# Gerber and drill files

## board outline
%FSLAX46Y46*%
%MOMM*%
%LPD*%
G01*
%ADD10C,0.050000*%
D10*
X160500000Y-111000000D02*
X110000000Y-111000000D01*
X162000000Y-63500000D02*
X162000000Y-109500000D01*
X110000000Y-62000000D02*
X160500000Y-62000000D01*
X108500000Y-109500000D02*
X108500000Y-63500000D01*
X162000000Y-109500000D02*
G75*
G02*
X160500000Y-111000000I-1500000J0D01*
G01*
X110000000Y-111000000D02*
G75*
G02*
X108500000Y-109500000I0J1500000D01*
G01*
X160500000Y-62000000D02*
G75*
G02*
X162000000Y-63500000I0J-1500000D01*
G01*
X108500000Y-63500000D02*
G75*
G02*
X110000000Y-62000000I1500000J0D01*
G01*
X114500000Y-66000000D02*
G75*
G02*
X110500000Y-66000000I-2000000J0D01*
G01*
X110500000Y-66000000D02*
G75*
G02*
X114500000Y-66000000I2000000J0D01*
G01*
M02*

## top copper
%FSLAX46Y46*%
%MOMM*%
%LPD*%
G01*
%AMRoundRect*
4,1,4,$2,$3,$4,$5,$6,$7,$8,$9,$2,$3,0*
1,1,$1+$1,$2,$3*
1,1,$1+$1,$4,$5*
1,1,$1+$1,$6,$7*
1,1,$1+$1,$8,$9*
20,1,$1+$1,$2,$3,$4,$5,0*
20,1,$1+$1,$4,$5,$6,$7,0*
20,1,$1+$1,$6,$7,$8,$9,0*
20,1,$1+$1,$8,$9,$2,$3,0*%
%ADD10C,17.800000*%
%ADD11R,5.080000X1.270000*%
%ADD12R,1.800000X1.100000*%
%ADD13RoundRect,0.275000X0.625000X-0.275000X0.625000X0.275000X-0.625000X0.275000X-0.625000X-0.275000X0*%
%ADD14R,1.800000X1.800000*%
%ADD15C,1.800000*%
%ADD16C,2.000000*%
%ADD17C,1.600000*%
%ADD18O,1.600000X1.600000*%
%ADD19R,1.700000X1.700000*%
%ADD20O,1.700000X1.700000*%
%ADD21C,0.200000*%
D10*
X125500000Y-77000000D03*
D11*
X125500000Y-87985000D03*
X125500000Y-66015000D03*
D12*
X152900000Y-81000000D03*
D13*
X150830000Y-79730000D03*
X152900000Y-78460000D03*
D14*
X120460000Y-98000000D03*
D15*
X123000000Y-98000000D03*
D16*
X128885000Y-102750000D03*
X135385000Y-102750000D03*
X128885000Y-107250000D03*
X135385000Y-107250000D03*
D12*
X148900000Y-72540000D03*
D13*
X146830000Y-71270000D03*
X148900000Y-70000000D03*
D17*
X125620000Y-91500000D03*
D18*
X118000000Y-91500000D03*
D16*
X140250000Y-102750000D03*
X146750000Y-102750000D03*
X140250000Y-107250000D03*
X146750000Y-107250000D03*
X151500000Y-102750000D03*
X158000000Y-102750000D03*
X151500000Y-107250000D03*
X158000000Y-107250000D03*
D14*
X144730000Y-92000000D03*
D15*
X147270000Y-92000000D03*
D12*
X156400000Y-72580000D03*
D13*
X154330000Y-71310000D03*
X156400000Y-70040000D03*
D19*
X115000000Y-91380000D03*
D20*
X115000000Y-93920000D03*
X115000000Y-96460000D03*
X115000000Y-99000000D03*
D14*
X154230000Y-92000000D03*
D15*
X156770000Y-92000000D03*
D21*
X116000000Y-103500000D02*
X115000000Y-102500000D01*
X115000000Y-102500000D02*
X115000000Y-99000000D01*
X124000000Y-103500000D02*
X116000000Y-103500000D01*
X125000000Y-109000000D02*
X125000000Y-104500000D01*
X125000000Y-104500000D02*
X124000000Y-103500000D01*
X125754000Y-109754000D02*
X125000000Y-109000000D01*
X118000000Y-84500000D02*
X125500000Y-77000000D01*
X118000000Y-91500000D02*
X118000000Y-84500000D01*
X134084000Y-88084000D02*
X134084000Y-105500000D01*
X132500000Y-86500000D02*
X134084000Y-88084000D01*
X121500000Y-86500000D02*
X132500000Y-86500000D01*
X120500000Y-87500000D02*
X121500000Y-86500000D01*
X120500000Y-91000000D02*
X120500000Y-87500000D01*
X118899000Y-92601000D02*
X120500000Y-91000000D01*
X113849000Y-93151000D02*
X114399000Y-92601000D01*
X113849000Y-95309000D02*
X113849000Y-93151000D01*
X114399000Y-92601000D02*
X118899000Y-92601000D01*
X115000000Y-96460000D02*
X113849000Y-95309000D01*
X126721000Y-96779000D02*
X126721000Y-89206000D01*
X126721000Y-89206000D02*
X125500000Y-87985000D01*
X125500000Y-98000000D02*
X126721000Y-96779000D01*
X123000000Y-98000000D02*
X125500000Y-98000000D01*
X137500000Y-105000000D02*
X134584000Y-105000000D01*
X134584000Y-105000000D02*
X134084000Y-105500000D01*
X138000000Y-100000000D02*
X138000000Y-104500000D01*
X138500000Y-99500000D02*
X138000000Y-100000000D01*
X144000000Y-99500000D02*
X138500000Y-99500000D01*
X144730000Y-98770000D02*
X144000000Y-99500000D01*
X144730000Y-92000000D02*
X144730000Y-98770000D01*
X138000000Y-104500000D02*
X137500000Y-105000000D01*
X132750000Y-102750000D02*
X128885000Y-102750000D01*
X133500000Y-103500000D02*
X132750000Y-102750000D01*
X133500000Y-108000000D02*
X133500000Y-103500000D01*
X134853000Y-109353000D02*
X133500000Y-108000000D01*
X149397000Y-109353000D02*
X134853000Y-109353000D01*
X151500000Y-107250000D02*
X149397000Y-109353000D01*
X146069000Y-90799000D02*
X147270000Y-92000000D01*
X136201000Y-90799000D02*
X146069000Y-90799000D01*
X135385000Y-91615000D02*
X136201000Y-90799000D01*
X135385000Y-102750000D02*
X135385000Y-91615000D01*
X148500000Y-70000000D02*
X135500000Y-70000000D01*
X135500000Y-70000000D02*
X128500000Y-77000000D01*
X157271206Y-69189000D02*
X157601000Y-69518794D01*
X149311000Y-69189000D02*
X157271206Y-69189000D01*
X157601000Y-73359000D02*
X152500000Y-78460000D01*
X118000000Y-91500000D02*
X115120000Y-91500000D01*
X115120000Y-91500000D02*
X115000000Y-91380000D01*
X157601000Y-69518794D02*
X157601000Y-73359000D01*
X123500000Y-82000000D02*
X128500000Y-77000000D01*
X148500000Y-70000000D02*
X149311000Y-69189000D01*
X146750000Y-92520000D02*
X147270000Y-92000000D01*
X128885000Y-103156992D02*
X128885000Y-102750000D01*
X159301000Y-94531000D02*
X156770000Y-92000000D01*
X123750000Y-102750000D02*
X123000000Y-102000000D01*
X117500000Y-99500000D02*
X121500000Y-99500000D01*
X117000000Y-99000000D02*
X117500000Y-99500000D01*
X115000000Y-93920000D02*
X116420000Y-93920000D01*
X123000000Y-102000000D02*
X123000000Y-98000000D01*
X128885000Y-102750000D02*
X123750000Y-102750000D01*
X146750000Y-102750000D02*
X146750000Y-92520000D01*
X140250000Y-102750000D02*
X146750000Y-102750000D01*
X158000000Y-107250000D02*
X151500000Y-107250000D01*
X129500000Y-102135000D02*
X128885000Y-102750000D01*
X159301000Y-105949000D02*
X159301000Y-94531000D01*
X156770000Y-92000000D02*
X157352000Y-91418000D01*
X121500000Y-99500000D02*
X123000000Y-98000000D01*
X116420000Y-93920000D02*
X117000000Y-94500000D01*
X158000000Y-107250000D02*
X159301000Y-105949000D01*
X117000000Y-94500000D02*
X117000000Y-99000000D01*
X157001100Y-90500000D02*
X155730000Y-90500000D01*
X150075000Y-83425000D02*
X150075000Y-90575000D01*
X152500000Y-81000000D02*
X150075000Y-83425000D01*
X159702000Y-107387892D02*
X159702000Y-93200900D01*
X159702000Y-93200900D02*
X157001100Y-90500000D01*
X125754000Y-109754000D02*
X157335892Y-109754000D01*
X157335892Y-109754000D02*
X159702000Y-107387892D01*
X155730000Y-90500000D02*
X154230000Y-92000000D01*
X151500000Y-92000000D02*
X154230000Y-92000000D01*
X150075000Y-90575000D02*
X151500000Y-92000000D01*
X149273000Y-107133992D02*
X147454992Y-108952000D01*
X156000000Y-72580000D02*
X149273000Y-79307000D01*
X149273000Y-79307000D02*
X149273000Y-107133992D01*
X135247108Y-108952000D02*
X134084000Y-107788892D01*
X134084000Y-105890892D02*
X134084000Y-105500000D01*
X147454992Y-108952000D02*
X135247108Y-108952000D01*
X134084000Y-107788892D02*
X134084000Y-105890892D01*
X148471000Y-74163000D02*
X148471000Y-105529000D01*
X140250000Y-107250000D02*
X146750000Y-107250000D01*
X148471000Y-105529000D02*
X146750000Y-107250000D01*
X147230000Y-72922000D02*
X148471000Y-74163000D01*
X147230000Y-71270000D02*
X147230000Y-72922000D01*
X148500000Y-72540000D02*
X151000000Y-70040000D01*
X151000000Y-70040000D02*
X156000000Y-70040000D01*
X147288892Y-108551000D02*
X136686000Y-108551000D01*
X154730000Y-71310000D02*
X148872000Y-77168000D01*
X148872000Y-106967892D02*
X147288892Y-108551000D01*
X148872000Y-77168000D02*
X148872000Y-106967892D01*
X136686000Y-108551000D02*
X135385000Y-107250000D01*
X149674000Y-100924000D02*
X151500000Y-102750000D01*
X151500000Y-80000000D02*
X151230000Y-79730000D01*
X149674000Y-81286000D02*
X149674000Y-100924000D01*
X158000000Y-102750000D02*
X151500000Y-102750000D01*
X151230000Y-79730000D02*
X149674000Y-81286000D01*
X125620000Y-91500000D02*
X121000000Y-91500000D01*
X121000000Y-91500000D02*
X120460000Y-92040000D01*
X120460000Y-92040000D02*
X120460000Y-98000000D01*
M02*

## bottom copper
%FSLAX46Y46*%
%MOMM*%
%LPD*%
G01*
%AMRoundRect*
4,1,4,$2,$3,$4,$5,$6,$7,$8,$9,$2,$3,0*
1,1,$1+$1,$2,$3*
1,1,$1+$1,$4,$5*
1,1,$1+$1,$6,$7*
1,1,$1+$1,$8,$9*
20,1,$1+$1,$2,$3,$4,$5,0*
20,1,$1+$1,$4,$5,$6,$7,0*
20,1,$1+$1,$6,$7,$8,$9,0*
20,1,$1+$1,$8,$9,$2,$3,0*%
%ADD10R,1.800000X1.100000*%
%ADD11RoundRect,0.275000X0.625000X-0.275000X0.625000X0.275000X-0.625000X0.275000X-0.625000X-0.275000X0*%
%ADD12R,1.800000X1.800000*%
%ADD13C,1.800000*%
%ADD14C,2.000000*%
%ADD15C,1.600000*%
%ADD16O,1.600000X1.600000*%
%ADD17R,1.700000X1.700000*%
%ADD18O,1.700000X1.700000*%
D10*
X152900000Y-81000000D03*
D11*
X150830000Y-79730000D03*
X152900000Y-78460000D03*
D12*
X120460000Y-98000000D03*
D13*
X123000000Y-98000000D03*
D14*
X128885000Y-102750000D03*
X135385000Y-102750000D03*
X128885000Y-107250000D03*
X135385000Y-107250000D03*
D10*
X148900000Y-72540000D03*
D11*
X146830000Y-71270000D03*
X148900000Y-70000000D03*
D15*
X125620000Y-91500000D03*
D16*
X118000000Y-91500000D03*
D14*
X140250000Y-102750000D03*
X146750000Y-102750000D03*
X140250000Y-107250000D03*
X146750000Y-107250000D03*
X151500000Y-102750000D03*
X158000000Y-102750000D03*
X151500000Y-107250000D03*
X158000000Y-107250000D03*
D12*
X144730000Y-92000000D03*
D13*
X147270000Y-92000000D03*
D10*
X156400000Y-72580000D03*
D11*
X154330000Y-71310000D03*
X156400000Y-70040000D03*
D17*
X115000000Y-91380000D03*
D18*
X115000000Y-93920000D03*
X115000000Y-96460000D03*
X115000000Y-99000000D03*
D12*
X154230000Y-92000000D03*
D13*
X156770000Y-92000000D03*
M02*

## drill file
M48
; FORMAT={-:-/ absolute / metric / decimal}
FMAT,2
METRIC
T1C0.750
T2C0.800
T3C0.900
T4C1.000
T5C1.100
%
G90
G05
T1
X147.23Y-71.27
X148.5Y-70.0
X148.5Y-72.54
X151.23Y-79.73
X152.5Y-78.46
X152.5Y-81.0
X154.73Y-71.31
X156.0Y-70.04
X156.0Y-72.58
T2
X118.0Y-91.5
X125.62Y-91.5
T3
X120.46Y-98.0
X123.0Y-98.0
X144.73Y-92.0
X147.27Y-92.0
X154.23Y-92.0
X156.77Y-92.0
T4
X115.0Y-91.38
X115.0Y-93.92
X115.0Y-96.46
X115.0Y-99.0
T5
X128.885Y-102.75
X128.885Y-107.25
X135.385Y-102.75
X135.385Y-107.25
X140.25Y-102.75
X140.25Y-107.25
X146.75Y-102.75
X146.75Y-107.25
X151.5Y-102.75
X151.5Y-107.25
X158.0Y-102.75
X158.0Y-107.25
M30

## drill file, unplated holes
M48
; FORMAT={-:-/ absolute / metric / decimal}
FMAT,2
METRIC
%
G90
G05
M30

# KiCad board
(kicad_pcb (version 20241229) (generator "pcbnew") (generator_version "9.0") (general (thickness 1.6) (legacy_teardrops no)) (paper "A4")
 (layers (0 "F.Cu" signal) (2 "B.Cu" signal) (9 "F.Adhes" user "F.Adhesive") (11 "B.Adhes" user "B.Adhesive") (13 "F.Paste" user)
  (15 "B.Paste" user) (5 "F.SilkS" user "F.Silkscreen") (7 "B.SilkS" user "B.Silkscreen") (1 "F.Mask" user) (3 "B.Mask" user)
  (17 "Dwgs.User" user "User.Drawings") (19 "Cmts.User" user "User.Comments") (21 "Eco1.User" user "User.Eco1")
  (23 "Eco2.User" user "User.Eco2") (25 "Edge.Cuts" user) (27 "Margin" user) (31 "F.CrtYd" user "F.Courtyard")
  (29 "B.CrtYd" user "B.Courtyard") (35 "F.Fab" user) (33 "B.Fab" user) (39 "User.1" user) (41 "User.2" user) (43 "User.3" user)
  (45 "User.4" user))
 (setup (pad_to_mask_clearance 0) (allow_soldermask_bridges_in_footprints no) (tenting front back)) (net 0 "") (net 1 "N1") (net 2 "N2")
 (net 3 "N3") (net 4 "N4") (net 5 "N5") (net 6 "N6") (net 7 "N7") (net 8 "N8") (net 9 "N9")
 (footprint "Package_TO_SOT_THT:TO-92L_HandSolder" (layer "F.Cu") (at 152.5 81 90)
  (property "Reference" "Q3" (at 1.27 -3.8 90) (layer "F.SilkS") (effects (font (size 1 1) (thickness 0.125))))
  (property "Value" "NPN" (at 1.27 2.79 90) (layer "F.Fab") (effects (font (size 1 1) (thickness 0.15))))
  (pad "1" thru_hole rect (at 0 0 90) (size 1.1 1.8) (drill 0.75 (offset 0 0.4)) (layers "*.Cu" "*.Mask") (remove_unused_layers no)
   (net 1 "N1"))
  (pad "2" thru_hole roundrect (at 1.27 -1.27 90) (size 1.1 1.8) (drill 0.75 (offset 0 -0.4)) (layers "*.Cu" "*.Mask")
   (remove_unused_layers no) (roundrect_rratio 0.25) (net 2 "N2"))
  (pad "3" thru_hole roundrect (at 2.54 0 90) (size 1.1 1.8) (drill 0.75 (offset 0 0.4)) (layers "*.Cu" "*.Mask") (remove_unused_layers no)
   (roundrect_rratio 0.25) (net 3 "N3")))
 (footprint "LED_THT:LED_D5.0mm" (layer "F.Cu") (at 120.46 98)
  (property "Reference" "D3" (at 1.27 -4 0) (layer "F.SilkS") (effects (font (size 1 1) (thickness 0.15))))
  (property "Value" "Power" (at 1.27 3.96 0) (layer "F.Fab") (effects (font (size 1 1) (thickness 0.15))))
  (pad "1" thru_hole rect (at 0 0) (size 1.8 1.8) (drill 0.9) (layers "*.Cu" "*.Mask") (remove_unused_layers no) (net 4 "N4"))
  (pad "2" thru_hole circle (at 2.54 0) (size 1.8 1.8) (drill 0.9) (layers "*.Cu" "*.Mask") (remove_unused_layers no) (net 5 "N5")))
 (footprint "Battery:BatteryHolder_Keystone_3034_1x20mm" (layer "F.Cu") (at 125.5 77 -90)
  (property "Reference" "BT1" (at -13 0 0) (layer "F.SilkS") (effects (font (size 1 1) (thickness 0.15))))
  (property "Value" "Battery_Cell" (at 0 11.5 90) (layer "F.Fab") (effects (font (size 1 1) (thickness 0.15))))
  (pad "1" smd rect (at -10.985 0 270) (size 1.27 5.08) (layers "F.Cu" "F.Mask" "F.Paste") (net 5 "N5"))
  (pad "1" smd rect (at 10.985 0 270) (size 1.27 5.08) (layers "F.Cu" "F.Mask" "F.Paste") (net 5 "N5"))
  (pad "2" smd circle (at 0 0 270) (size 17.8 17.8) (layers "F.Cu" "F.Mask") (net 3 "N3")))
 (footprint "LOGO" (layer "F.Cu") (at 140 68)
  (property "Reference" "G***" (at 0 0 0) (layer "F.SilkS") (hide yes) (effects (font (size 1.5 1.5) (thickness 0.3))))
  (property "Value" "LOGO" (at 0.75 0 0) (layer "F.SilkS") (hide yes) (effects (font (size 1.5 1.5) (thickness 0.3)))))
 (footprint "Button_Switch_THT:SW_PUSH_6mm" (layer "F.Cu") (at 128.885 102.75)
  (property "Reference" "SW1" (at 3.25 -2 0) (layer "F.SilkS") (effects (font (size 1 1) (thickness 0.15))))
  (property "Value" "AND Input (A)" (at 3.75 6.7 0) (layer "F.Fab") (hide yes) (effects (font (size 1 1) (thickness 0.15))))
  (pad "1" thru_hole circle (at 0 0 90) (size 2 2) (drill 1.1) (layers "*.Cu" "*.Mask") (remove_unused_layers no) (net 5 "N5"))
  (pad "1" thru_hole circle (at 6.5 0 90) (size 2 2) (drill 1.1) (layers "*.Cu" "*.Mask") (remove_unused_layers no) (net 5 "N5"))
  (pad "2" thru_hole circle (at 0 4.5 90) (size 2 2) (drill 1.1) (layers "*.Cu" "*.Mask") (remove_unused_layers no) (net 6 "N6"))
  (pad "2" thru_hole circle (at 6.5 4.5 90) (size 2 2) (drill 1.1) (layers "*.Cu" "*.Mask") (remove_unused_layers no) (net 6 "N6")))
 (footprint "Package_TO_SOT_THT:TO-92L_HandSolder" (layer "F.Cu") (at 148.5 72.54 90)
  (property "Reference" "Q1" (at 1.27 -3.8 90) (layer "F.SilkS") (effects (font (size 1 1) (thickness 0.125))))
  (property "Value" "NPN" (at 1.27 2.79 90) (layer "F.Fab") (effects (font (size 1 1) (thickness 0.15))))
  (pad "1" thru_hole rect (at 0 0 90) (size 1.1 1.8) (drill 0.75 (offset 0 0.4)) (layers "*.Cu" "*.Mask") (remove_unused_layers no)
   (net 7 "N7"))
  (pad "2" thru_hole roundrect (at 1.27 -1.27 90) (size 1.1 1.8) (drill 0.75 (offset 0 -0.4)) (layers "*.Cu" "*.Mask")
   (remove_unused_layers no) (roundrect_rratio 0.25) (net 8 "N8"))
  (pad "3" thru_hole roundrect (at 2.54 0 90) (size 1.1 1.8) (drill 0.75 (offset 0 0.4)) (layers "*.Cu" "*.Mask") (remove_unused_layers no)
   (roundrect_rratio 0.25) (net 3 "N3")))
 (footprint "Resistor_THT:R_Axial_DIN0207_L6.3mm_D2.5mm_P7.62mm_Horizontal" (layer "F.Cu") (at 125.62 91.5 180)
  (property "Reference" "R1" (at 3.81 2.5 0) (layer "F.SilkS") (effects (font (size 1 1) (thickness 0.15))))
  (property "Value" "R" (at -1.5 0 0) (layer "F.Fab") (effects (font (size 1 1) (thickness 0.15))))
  (pad "1" thru_hole circle (at 0 0 180) (size 1.6 1.6) (drill 0.8) (layers "*.Cu" "*.Mask") (remove_unused_layers no) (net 4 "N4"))
  (pad "2" thru_hole oval (at 7.62 0 180) (size 1.6 1.6) (drill 0.8) (layers "*.Cu" "*.Mask") (remove_unused_layers no) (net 3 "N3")))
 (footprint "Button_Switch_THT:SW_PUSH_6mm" (layer "F.Cu") (at 140.25 102.75)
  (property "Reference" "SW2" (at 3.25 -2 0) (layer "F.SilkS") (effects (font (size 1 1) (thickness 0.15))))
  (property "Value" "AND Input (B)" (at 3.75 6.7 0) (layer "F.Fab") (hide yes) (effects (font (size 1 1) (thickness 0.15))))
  (pad "1" thru_hole circle (at 0 0 90) (size 2 2) (drill 1.1) (layers "*.Cu" "*.Mask") (remove_unused_layers no) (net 5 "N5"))
  (pad "1" thru_hole circle (at 6.5 0 90) (size 2 2) (drill 1.1) (layers "*.Cu" "*.Mask") (remove_unused_layers no) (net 5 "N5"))
  (pad "2" thru_hole circle (at 0 4.5 90) (size 2 2) (drill 1.1) (layers "*.Cu" "*.Mask") (remove_unused_layers no) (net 8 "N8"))
  (pad "2" thru_hole circle (at 6.5 4.5 90) (size 2 2) (drill 1.1) (layers "*.Cu" "*.Mask") (remove_unused_layers no) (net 8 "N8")))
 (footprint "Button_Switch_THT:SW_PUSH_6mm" (layer "F.Cu") (at 151.5 102.75)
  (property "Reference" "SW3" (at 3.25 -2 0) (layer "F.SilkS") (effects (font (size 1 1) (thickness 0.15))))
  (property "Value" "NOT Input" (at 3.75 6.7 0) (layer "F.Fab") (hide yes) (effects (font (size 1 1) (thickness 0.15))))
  (pad "1" thru_hole circle (at 0 0 90) (size 2 2) (drill 1.1) (layers "*.Cu" "*.Mask") (remove_unused_layers no) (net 2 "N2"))
  (pad "1" thru_hole circle (at 6.5 0 90) (size 2 2) (drill 1.1) (layers "*.Cu" "*.Mask") (remove_unused_layers no) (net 2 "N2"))
  (pad "2" thru_hole circle (at 0 4.5 90) (size 2 2) (drill 1.1) (layers "*.Cu" "*.Mask") (remove_unused_layers no) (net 5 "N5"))
  (pad "2" thru_hole circle (at 6.5 4.5 90) (size 2 2) (drill 1.1) (layers "*.Cu" "*.Mask") (remove_unused_layers no) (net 5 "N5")))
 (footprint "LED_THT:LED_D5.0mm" (layer "F.Cu") (at 144.73 92)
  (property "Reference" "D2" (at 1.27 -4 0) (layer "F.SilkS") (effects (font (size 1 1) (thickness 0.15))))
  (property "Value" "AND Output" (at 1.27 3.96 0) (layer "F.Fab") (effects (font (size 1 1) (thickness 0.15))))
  (pad "1" thru_hole rect (at 0 0) (size 1.8 1.8) (drill 0.9) (layers "*.Cu" "*.Mask") (remove_unused_layers no) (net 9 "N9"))
  (pad "2" thru_hole circle (at 2.54 0) (size 1.8 1.8) (drill 0.9) (layers "*.Cu" "*.Mask") (remove_unused_layers no) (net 5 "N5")))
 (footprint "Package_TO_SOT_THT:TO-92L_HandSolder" (layer "F.Cu") (at 156 72.58 90)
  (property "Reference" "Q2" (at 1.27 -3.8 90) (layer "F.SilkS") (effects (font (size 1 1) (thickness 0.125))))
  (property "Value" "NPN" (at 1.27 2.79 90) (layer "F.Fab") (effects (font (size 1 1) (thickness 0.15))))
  (pad "1" thru_hole rect (at 0 0 90) (size 1.1 1.8) (drill 0.75 (offset 0 0.4)) (layers "*.Cu" "*.Mask") (remove_unused_layers no)
   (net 9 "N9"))
  (pad "2" thru_hole roundrect (at 1.27 -1.27 90) (size 1.1 1.8) (drill 0.75 (offset 0 -0.4)) (layers "*.Cu" "*.Mask")
   (remove_unused_layers no) (roundrect_rratio 0.25) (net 6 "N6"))
  (pad "3" thru_hole roundrect (at 2.54 0 90) (size 1.1 1.8) (drill 0.75 (offset 0 0.4)) (layers "*.Cu" "*.Mask") (remove_unused_layers no)
   (roundrect_rratio 0.25) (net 7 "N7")))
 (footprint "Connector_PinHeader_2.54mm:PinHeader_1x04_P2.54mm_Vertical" (layer "F.Cu") (at 115 91.38)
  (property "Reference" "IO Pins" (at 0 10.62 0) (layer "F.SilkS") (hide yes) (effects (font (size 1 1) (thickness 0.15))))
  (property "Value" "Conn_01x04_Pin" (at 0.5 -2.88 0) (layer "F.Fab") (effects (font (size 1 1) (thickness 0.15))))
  (pad "1" thru_hole rect (at 0 0) (size 1.7 1.7) (drill 1) (layers "*.Cu" "*.Mask") (remove_unused_layers no) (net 3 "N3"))
  (pad "2" thru_hole oval (at 0 2.54) (size 1.7 1.7) (drill 1) (layers "*.Cu" "*.Mask") (remove_unused_layers no) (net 5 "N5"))
  (pad "3" thru_hole oval (at 0 5.08) (size 1.7 1.7) (drill 1) (layers "*.Cu" "*.Mask") (remove_unused_layers no) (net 9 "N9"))
  (pad "4" thru_hole oval (at 0 7.62) (size 1.7 1.7) (drill 1) (layers "*.Cu" "*.Mask") (remove_unused_layers no) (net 1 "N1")))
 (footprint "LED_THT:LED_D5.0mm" (layer "F.Cu") (at 154.23 92)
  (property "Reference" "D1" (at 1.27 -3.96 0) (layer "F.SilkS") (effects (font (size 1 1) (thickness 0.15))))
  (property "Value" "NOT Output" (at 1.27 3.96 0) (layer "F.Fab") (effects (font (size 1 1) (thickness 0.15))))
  (pad "1" thru_hole rect (at 0 0) (size 1.8 1.8) (drill 0.9) (layers "*.Cu" "*.Mask") (remove_unused_layers no) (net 1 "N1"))
  (pad "2" thru_hole circle (at 2.54 0) (size 1.8 1.8) (drill 0.9) (layers "*.Cu" "*.Mask") (remove_unused_layers no) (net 5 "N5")))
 (gr_line (start 108.5 109.5) (end 108.5 63.5) (stroke (width 0.05) (type default)) (layer "Edge.Cuts"))
 (gr_circle (center 112.5 66) (end 112.5 68) (stroke (width 0.05) (type default)) (fill no) (layer "Edge.Cuts"))
 (gr_arc (start 110 111) (mid 108.93934 110.56066) (end 108.5 109.5) (stroke (width 0.05) (type default)) (layer "Edge.Cuts"))
 (gr_arc (start 160.5 62) (mid 161.56066 62.43934) (end 162 63.5) (stroke (width 0.05) (type default)) (layer "Edge.Cuts"))
 (gr_line (start 162 63.5) (end 162 109.5) (stroke (width 0.05) (type default)) (layer "Edge.Cuts"))
 (gr_line (start 110 62) (end 160.5 62) (stroke (width 0.05) (type default)) (layer "Edge.Cuts"))
 (gr_arc (start 108.5 63.5) (mid 108.93934 62.43934) (end 110 62) (stroke (width 0.05) (type default)) (layer "Edge.Cuts"))
 (gr_arc (start 162 109.5) (mid 161.56066 110.56066) (end 160.5 111) (stroke (width 0.05) (type default)) (layer "Edge.Cuts"))
 (gr_line (start 160.5 111) (end 110 111) (stroke (width 0.05) (type default)) (layer "Edge.Cuts"))
 (segment (start 118 84.5) (end 125.5 77) (width 0.2) (layer "F.Cu") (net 3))
 (segment (start 148.5 70) (end 135.5 70) (width 0.2) (layer "F.Cu") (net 3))
 (segment (start 135.5 70) (end 128.5 77) (width 0.2) (layer "F.Cu") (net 3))
 (segment (start 157.271206 69.189) (end 157.601 69.518794) (width 0.2) (layer "F.Cu") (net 3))
 (segment (start 149.311 69.189) (end 157.271206 69.189) (width 0.2) (layer "F.Cu") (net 3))
 (segment (start 157.601 73.359) (end 152.5 78.46) (width 0.2) (layer "F.Cu") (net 3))
 (segment (start 118 91.5) (end 115.12 91.5) (width 0.2) (layer "F.Cu") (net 3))
 (segment (start 115.12 91.5) (end 115 91.38) (width 0.2) (layer "F.Cu") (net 3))
 (segment (start 157.601 69.518794) (end 157.601 73.359) (width 0.2) (layer "F.Cu") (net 3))
 (segment (start 118 91.5) (end 118 84.5) (width 0.2) (layer "F.Cu") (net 3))
 (segment (start 123.5 82) (end 128.5 77) (width 0.2) (layer "F.Cu") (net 3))
 (segment (start 148.5 70) (end 149.311 69.189) (width 0.2) (layer "F.Cu") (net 3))
 (segment (start 125.5 98) (end 126.721 96.779) (width 0.2) (layer "F.Cu") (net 5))
 (segment (start 151.5 107.25) (end 149.397 109.353) (width 0.2) (layer "F.Cu") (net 5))
 (segment (start 146.75 92.52) (end 147.27 92) (width 0.2) (layer "F.Cu") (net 5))
 (segment (start 128.885 103.156992) (end 128.885 102.75) (width 0.2) (layer "F.Cu") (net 5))
 (segment (start 159.301 94.531) (end 156.77 92) (width 0.2) (layer "F.Cu") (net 5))
 (segment (start 133.5 103.5) (end 132.75 102.75) (width 0.2) (layer "F.Cu") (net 5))
 (segment (start 132.75 102.75) (end 128.885 102.75) (width 0.2) (layer "F.Cu") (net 5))
 (segment (start 123 98) (end 125.5 98) (width 0.2) (layer "F.Cu") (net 5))
 (segment (start 123.75 102.75) (end 123 102) (width 0.2) (layer "F.Cu") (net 5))
 (segment (start 117.5 99.5) (end 121.5 99.5) (width 0.2) (layer "F.Cu") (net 5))
 (segment (start 133.5 108) (end 133.5 103.5) (width 0.2) (layer "F.Cu") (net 5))
 (segment (start 135.385 91.615) (end 136.201 90.799) (width 0.2) (layer "F.Cu") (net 5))
 (segment (start 117 99) (end 117.5 99.5) (width 0.2) (layer "F.Cu") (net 5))
 (segment (start 115 93.92) (end 116.42 93.92) (width 0.2) (layer "F.Cu") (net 5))
 (segment (start 123 102) (end 123 98) (width 0.2) (layer "F.Cu") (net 5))
 (segment (start 126.721 96.779) (end 126.721 89.206) (width 0.2) (layer "F.Cu") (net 5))
 (segment (start 128.885 102.75) (end 123.75 102.75) (width 0.2) (layer "F.Cu") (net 5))
 (segment (start 146.75 102.75) (end 146.75 92.52) (width 0.2) (layer "F.Cu") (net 5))
 (segment (start 140.25 102.75) (end 146.75 102.75) (width 0.2) (layer "F.Cu") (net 5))
 (segment (start 146.069 90.799) (end 147.27 92) (width 0.2) (layer "F.Cu") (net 5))
 (segment (start 158 107.25) (end 151.5 107.25) (width 0.2) (layer "F.Cu") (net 5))
 (segment (start 136.201 90.799) (end 146.069 90.799) (width 0.2) (layer "F.Cu") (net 5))
 (segment (start 135.385 102.75) (end 135.385 91.615) (width 0.2) (layer "F.Cu") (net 5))
 (segment (start 129.5 102.135) (end 128.885 102.75) (width 0.2) (layer "F.Cu") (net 5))
 (segment (start 134.853 109.353) (end 133.5 108) (width 0.2) (layer "F.Cu") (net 5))
 (segment (start 159.301 105.949) (end 159.301 94.531) (width 0.2) (layer "F.Cu") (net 5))
 (segment (start 149.397 109.353) (end 134.853 109.353) (width 0.2) (layer "F.Cu") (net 5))
 (segment (start 156.77 92) (end 157.352 91.418) (width 0.2) (layer "F.Cu") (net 5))
 (segment (start 121.5 99.5) (end 123 98) (width 0.2) (layer "F.Cu") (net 5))
 (segment (start 116.42 93.92) (end 117 94.5) (width 0.2) (layer "F.Cu") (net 5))
 (segment (start 158 107.25) (end 159.301 105.949) (width 0.2) (layer "F.Cu") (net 5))
 (segment (start 126.721 89.206) (end 125.5 87.985) (width 0.2) (layer "F.Cu") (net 5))
 (segment (start 117 94.5) (end 117 99) (width 0.2) (layer "F.Cu") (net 5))
 (segment (start 115 102.5) (end 115 99) (width 0.2) (layer "F.Cu") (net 1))
 (segment (start 157.0011 90.5) (end 155.73 90.5) (width 0.2) (layer "F.Cu") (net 1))
 (segment (start 150.075 83.425) (end 150.075 90.575) (width 0.2) (layer "F.Cu") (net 1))
 (segment (start 125 104.5) (end 124 103.5) (width 0.2) (layer "F.Cu") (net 1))
 (segment (start 124 103.5) (end 116 103.5) (width 0.2) (layer "F.Cu") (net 1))
 (segment (start 152.5 81) (end 150.075 83.425) (width 0.2) (layer "F.Cu") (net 1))
 (segment (start 125 109) (end 125 104.5) (width 0.2) (layer "F.Cu") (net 1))
 (segment (start 159.702 107.387892) (end 159.702 93.2009) (width 0.2) (layer "F.Cu") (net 1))
 (segment (start 159.702 93.2009) (end 157.0011 90.5) (width 0.2) (layer "F.Cu") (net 1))
 (segment (start 125.754 109.754) (end 125 109) (width 0.2) (layer "F.Cu") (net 1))
 (segment (start 125.754 109.754) (end 157.335892 109.754) (width 0.2) (layer "F.Cu") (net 1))
 (segment (start 157.335892 109.754) (end 159.702 107.387892) (width 0.2) (layer "F.Cu") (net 1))
 (segment (start 116 103.5) (end 115 102.5) (width 0.2) (layer "F.Cu") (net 1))
 (segment (start 155.73 90.5) (end 154.23 92) (width 0.2) (layer "F.Cu") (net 1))
 (segment (start 151.5 92) (end 154.23 92) (width 0.2) (layer "F.Cu") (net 1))
 (segment (start 150.075 90.575) (end 151.5 92) (width 0.2) (layer "F.Cu") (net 1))
 (segment (start 114.399 92.601) (end 118.899 92.601) (width 0.2) (layer "F.Cu") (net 9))
 (segment (start 149.273 107.133992) (end 147.454992 108.952) (width 0.2) (layer "F.Cu") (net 9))
 (segment (start 118.899 92.601) (end 120.5 91) (width 0.2) (layer "F.Cu") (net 9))
 (segment (start 120.5 87.5) (end 121.5 86.5) (width 0.2) (layer "F.Cu") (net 9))
 (segment (start 137.5 105) (end 134.584 105) (width 0.2) (layer "F.Cu") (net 9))
 (segment (start 121.5 86.5) (end 132.5 86.5) (width 0.2) (layer "F.Cu") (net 9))
 (segment (start 144.73 92) (end 144.73 98.77) (width 0.2) (layer "F.Cu") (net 9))
 (segment (start 138 104.5) (end 137.5 105) (width 0.2) (layer "F.Cu") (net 9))
 (segment (start 156 72.58) (end 149.273 79.307) (width 0.2) (layer "F.Cu") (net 9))
 (segment (start 149.273 79.307) (end 149.273 107.133992) (width 0.2) (layer "F.Cu") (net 9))
 (segment (start 115 96.46) (end 113.849 95.309) (width 0.2) (layer "F.Cu") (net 9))
 (segment (start 120.5 91) (end 120.5 87.5) (width 0.2) (layer "F.Cu") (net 9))
 (segment (start 138.5 99.5) (end 138 100) (width 0.2) (layer "F.Cu") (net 9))
 (segment (start 113.849 95.309) (end 113.849 93.151) (width 0.2) (layer "F.Cu") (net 9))
 (segment (start 132.5 86.5) (end 134.084 88.084) (width 0.2) (layer "F.Cu") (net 9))
 (segment (start 144 99.5) (end 138.5 99.5) (width 0.2) (layer "F.Cu") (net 9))
 (segment (start 138 100) (end 138 104.5) (width 0.2) (layer "F.Cu") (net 9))
 (segment (start 135.247108 108.952) (end 134.084 107.788892) (width 0.2) (layer "F.Cu") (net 9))
 (segment (start 144.73 98.77) (end 144 99.5) (width 0.2) (layer "F.Cu") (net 9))
 (segment (start 134.084 105.890892) (end 134.084 105.5) (width 0.2) (layer "F.Cu") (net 9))
 (segment (start 147.454992 108.952) (end 135.247108 108.952) (width 0.2) (layer "F.Cu") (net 9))
 (segment (start 134.584 105) (end 134.084 105.5) (width 0.2) (layer "F.Cu") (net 9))
 (segment (start 134.084 88.084) (end 134.084 105.5) (width 0.2) (layer "F.Cu") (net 9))
 (segment (start 113.849 93.151) (end 114.399 92.601) (width 0.2) (layer "F.Cu") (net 9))
 (segment (start 134.084 107.788892) (end 134.084 105.890892) (width 0.2) (layer "F.Cu") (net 9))
 (segment (start 148.471 74.163) (end 148.471 105.529) (width 0.2) (layer "F.Cu") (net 8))
 (segment (start 140.25 107.25) (end 146.75 107.25) (width 0.2) (layer "F.Cu") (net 8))
 (segment (start 148.471 105.529) (end 146.75 107.25) (width 0.2) (layer "F.Cu") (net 8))
 (segment (start 147.23 72.922) (end 148.471 74.163) (width 0.2) (layer "F.Cu") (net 8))
 (segment (start 147.23 71.27) (end 147.23 72.922) (width 0.2) (layer "F.Cu") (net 8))
 (segment (start 148.5 72.54) (end 151 70.04) (width 0.2) (layer "F.Cu") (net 7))
 (segment (start 151 70.04) (end 156 70.04) (width 0.2) (layer "F.Cu") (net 7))
 (segment (start 147.288892 108.551) (end 136.686 108.551) (width 0.2) (layer "F.Cu") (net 6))
 (segment (start 154.73 71.31) (end 148.872 77.168) (width 0.2) (layer "F.Cu") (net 6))
 (segment (start 148.872 106.967892) (end 147.288892 108.551) (width 0.2) (layer "F.Cu") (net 6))
 (segment (start 148.872 77.168) (end 148.872 106.967892) (width 0.2) (layer "F.Cu") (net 6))
 (segment (start 136.686 108.551) (end 135.385 107.25) (width 0.2) (layer "F.Cu") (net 6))
 (segment (start 149.674 100.924) (end 151.5 102.75) (width 0.2) (layer "F.Cu") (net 2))
 (segment (start 151.5 80) (end 151.23 79.73) (width 0.2) (layer "F.Cu") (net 2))
 (segment (start 149.674 81.286) (end 149.674 100.924) (width 0.2) (layer "F.Cu") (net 2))
 (segment (start 158 102.75) (end 151.5 102.75) (width 0.2) (layer "F.Cu") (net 2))
 (segment (start 151.23 79.73) (end 149.674 81.286) (width 0.2) (layer "F.Cu") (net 2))
 (segment (start 125.62 91.5) (end 121 91.5) (width 0.2) (layer "F.Cu") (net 4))
 (segment (start 121 91.5) (end 120.46 92.04) (width 0.2) (layer "F.Cu") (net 4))
 (segment (start 120.46 92.04) (end 120.46 98) (width 0.2) (layer "F.Cu") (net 4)))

